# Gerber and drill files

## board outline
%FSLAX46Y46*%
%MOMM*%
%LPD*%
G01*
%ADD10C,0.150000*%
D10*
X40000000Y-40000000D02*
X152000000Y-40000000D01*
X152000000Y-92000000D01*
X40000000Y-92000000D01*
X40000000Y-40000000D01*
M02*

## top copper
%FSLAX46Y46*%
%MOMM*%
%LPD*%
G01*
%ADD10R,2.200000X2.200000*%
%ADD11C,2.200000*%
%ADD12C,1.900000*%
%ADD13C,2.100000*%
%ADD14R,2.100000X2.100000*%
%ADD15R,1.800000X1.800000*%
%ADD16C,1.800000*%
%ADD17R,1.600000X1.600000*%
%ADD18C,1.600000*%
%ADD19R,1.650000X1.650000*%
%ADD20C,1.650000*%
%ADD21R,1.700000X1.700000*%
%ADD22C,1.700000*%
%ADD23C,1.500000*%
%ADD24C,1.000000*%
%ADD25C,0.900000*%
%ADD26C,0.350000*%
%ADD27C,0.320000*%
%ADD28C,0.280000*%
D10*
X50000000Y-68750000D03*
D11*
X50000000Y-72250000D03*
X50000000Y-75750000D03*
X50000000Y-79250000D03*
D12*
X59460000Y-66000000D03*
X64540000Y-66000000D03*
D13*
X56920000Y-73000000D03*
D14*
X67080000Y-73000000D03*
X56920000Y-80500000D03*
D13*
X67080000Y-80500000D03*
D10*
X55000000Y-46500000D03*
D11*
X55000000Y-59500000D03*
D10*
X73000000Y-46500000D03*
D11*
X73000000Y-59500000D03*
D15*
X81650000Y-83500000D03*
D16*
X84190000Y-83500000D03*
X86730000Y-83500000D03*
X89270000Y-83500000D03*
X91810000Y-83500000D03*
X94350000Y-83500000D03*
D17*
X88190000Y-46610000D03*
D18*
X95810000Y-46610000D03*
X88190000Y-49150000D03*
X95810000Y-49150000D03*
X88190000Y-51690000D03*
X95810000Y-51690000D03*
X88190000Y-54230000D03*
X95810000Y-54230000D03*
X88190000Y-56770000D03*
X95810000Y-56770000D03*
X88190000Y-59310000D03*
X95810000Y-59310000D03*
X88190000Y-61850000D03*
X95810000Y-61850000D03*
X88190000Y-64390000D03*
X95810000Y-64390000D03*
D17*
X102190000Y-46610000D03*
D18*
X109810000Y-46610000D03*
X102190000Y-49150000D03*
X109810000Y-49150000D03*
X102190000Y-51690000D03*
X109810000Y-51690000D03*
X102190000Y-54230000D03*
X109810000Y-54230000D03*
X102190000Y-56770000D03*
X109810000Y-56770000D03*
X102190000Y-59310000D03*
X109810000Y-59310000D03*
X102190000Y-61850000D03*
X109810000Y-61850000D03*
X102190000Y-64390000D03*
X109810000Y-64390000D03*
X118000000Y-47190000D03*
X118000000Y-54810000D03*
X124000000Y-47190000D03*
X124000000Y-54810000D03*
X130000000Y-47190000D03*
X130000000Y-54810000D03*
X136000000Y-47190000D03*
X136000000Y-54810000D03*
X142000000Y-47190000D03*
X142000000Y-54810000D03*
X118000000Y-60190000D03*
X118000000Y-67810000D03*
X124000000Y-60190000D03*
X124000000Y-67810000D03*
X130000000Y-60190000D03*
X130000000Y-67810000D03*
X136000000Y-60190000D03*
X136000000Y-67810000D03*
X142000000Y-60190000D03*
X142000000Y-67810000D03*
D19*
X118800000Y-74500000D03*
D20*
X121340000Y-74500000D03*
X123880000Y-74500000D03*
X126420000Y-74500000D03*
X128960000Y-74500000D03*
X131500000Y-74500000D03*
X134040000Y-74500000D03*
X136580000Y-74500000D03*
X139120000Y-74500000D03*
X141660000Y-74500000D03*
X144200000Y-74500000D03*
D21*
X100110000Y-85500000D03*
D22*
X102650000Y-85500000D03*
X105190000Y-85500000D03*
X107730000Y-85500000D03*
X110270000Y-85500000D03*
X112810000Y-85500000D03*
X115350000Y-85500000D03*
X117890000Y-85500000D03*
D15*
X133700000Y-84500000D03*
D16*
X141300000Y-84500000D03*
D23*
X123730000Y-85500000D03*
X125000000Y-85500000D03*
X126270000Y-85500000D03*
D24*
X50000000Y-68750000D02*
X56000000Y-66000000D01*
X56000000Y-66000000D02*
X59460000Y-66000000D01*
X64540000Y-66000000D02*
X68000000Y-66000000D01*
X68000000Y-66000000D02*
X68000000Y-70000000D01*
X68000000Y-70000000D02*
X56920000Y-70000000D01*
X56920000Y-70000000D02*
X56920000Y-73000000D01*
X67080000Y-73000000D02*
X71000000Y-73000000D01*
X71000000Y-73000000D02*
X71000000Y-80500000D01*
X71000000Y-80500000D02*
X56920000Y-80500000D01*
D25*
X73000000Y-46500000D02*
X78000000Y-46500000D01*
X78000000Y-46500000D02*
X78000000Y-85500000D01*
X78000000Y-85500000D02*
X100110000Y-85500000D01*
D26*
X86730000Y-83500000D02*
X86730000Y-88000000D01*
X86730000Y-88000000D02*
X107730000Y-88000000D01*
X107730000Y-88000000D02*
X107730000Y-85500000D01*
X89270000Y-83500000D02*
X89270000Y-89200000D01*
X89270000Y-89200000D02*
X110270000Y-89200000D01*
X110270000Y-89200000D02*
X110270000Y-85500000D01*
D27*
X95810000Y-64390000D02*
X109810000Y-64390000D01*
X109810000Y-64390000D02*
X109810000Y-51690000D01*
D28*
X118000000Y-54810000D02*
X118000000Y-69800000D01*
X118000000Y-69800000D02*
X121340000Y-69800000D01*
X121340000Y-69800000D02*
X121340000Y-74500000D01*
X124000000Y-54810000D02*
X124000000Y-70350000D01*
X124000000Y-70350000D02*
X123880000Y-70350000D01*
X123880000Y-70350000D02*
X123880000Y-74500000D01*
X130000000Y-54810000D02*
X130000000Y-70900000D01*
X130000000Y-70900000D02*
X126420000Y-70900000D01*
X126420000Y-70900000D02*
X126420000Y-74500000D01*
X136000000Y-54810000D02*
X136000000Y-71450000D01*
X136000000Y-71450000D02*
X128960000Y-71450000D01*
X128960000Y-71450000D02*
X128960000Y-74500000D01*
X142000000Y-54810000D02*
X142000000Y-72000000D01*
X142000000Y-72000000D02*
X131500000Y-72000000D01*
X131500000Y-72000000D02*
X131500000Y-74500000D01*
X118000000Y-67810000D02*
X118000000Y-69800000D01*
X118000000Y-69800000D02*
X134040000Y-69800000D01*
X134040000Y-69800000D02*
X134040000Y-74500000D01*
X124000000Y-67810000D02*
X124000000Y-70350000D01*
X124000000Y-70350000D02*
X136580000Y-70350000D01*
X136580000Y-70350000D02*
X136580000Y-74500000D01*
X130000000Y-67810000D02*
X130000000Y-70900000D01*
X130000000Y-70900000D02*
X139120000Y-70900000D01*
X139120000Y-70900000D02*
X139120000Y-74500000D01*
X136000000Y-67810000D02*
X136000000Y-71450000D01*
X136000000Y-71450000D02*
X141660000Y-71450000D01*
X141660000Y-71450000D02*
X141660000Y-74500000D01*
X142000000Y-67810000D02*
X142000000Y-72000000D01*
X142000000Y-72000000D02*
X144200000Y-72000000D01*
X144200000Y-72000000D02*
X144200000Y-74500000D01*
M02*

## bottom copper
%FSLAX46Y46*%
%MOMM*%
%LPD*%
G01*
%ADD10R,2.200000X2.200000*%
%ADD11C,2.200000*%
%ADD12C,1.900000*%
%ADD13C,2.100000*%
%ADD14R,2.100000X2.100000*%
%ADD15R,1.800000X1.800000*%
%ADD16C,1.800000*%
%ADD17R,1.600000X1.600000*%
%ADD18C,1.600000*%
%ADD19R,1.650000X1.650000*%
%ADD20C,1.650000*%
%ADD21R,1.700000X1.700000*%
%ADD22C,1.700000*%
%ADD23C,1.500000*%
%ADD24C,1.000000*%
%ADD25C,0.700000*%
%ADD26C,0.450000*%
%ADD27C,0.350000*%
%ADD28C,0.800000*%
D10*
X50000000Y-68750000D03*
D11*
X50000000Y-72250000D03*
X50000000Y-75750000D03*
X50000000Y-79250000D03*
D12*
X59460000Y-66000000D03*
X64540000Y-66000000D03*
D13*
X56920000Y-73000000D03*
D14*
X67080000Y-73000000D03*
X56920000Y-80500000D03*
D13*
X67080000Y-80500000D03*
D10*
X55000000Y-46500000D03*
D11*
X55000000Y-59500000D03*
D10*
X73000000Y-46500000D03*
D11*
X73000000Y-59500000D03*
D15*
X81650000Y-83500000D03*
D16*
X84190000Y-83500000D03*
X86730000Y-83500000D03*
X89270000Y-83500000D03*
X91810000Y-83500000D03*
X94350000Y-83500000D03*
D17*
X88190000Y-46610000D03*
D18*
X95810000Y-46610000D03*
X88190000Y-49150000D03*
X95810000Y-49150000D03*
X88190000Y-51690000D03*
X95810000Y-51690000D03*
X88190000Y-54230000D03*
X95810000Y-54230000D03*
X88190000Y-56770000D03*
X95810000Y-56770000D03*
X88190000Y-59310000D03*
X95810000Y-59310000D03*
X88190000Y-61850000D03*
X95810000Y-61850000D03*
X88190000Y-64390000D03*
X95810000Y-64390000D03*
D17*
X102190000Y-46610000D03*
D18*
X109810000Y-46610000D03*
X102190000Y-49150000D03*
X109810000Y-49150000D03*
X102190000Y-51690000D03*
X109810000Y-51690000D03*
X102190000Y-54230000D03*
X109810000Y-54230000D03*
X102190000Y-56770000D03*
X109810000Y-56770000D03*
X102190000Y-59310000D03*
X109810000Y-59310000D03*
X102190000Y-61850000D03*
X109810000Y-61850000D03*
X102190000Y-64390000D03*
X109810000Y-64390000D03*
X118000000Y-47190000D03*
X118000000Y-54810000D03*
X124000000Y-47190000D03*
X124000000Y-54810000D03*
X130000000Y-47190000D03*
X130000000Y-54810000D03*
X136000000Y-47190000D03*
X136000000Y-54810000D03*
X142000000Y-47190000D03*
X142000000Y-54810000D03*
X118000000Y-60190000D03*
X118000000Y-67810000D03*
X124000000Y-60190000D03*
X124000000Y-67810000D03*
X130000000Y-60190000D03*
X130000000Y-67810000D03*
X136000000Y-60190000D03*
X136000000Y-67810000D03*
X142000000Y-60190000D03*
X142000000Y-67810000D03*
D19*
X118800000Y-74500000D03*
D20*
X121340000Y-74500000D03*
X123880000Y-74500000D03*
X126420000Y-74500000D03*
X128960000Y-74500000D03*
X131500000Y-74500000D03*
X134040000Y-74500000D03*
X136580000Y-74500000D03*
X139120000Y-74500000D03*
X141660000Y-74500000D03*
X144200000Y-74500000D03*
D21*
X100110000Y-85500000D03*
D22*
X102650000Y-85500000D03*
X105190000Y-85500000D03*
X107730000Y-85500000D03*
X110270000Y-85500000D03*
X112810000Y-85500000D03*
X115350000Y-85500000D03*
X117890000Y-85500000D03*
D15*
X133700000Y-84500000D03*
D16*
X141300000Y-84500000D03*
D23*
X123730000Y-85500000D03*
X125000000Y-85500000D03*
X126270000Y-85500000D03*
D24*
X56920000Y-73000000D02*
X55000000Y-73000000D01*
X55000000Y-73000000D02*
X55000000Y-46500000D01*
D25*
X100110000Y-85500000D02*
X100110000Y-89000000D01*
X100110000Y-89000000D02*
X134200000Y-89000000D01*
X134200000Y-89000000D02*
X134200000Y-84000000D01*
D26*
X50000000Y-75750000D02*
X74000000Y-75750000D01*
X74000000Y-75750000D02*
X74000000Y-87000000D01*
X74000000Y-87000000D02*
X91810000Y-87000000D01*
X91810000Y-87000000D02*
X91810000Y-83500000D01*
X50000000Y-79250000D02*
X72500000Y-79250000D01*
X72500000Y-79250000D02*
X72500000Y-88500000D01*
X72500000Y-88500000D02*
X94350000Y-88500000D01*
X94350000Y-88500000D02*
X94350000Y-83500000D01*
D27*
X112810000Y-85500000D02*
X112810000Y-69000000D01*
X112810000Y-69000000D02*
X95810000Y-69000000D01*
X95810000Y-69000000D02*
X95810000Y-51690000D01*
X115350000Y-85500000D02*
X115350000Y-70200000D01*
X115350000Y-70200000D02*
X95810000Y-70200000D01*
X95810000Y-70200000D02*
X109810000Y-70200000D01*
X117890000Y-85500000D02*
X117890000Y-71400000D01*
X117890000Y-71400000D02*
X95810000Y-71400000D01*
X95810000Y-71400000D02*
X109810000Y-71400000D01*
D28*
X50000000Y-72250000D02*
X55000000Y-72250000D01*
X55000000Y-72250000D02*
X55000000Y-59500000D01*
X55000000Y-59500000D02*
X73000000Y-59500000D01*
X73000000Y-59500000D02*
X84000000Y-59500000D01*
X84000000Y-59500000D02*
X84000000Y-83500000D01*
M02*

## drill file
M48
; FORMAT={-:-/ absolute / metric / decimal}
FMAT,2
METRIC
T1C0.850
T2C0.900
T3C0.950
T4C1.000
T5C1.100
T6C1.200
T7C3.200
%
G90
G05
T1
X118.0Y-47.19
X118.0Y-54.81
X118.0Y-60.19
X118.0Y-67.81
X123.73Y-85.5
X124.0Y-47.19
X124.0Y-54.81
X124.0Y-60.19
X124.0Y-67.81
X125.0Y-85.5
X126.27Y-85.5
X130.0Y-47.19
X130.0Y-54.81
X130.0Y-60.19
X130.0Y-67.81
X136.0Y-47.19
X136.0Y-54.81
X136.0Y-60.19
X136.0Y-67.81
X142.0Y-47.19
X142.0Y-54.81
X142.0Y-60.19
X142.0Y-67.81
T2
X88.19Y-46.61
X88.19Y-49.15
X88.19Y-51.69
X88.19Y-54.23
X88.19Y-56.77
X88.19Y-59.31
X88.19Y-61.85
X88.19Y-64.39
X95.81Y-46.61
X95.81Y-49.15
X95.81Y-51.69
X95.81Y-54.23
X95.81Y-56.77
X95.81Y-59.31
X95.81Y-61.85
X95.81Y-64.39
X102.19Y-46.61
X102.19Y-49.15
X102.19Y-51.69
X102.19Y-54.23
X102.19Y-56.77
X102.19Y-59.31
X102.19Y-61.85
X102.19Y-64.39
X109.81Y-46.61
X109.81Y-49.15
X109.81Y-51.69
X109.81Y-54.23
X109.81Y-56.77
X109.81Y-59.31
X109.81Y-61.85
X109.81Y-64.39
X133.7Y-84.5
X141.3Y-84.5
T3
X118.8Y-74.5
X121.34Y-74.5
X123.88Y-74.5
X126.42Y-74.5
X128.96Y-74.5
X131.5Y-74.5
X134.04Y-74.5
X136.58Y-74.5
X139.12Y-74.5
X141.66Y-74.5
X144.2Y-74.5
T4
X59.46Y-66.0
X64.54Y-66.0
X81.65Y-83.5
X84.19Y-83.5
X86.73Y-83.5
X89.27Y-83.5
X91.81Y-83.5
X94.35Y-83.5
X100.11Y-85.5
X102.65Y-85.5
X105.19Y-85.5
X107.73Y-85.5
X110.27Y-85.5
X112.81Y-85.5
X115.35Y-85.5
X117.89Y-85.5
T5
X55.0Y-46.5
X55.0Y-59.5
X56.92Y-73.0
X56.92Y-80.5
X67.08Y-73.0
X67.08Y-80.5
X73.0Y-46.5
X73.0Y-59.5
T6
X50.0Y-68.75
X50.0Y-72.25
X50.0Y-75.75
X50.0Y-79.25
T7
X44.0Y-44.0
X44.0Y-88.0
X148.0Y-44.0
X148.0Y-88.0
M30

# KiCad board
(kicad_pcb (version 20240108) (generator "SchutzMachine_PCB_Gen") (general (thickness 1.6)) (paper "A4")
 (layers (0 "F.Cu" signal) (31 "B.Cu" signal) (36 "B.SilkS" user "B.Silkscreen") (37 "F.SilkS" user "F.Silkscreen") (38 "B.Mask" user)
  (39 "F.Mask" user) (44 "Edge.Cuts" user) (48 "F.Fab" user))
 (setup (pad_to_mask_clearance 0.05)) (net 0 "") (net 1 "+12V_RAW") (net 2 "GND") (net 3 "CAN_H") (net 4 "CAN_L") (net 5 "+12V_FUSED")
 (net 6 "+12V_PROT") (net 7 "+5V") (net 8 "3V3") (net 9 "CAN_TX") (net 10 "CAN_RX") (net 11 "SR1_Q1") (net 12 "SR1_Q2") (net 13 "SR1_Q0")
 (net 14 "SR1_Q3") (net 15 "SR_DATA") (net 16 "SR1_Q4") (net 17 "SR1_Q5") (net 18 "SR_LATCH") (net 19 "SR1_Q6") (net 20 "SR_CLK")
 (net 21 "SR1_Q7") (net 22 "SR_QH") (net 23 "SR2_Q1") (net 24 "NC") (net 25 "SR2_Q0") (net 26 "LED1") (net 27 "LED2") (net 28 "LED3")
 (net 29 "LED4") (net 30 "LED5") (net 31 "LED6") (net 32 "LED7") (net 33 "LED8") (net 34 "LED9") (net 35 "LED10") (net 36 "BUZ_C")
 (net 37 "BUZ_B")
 (gr_rect (start 40.0 40.0) (end 152.0 92.0) (stroke (width 0.15) (type solid)) (fill none) (layer "Edge.Cuts"))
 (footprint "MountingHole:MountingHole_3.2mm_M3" (layer "F.Cu") (at 44.0 44.0)
  (pad "" np_thru_hole circle (at 0 0) (size 3.2 3.2) (drill 3.2) (layers "*.Cu" "*.Mask")))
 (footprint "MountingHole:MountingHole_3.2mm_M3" (layer "F.Cu") (at 148.0 44.0)
  (pad "" np_thru_hole circle (at 0 0) (size 3.2 3.2) (drill 3.2) (layers "*.Cu" "*.Mask")))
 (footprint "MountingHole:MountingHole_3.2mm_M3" (layer "F.Cu") (at 44.0 88.0)
  (pad "" np_thru_hole circle (at 0 0) (size 3.2 3.2) (drill 3.2) (layers "*.Cu" "*.Mask")))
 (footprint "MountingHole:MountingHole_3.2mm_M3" (layer "F.Cu") (at 148.0 88.0)
  (pad "" np_thru_hole circle (at 0 0) (size 3.2 3.2) (drill 3.2) (layers "*.Cu" "*.Mask")))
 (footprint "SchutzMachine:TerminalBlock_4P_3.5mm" (layer "F.Cu") (at 50.0 74.0 0)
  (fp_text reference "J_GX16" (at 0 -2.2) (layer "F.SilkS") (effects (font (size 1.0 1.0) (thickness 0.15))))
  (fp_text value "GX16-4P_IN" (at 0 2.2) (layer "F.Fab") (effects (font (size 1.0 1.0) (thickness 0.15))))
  (pad "1" thru_hole rect (at 0 -5.25) (size 2.2 2.2) (drill 1.2) (layers "*.Cu" "*.Mask") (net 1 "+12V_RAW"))
  (pad "2" thru_hole circle (at 0 -1.75) (size 2.2 2.2) (drill 1.2) (layers "*.Cu" "*.Mask") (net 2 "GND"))
  (pad "3" thru_hole circle (at 0 1.75) (size 2.2 2.2) (drill 1.2) (layers "*.Cu" "*.Mask") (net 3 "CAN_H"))
  (pad "4" thru_hole circle (at 0 5.25) (size 2.2 2.2) (drill 1.2) (layers "*.Cu" "*.Mask") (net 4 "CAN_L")))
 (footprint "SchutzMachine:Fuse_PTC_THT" (layer "F.Cu") (at 62.0 66.0 0)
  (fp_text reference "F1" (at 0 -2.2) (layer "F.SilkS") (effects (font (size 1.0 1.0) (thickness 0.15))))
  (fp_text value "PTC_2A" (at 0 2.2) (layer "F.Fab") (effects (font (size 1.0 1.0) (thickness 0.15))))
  (pad "1" thru_hole circle (at -2.54 0) (size 1.9 1.9) (drill 1.0) (layers "*.Cu" "*.Mask") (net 1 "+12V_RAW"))
  (pad "2" thru_hole circle (at 2.54 0) (size 1.9 1.9) (drill 1.0) (layers "*.Cu" "*.Mask") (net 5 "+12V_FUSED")))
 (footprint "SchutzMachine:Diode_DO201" (layer "F.Cu") (at 62.0 73.0 0)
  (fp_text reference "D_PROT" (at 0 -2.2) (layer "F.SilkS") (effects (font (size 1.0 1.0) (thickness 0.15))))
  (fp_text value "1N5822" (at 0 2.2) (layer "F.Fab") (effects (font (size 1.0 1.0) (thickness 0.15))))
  (pad "1" thru_hole circle (at -5.08 0) (size 2.1 2.1) (drill 1.1) (layers "*.Cu" "*.Mask") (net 5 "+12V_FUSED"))
  (pad "2" thru_hole rect (at 5.08 0) (size 2.1 2.1) (drill 1.1) (layers "*.Cu" "*.Mask") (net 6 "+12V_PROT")))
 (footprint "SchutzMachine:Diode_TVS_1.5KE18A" (layer "F.Cu") (at 62.0 80.5 0)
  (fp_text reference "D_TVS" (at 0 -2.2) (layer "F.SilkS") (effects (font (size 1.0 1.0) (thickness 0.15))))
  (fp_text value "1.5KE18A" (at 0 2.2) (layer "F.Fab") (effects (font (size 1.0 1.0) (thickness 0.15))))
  (pad "1" thru_hole rect (at -5.08 0) (size 2.1 2.1) (drill 1.1) (layers "*.Cu" "*.Mask") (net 6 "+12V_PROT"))
  (pad "2" thru_hole circle (at 5.08 0) (size 2.1 2.1) (drill 1.1) (layers "*.Cu" "*.Mask") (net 2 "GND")))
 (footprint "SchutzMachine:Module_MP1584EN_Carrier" (layer "F.Cu") (at 64.0 53.0 0)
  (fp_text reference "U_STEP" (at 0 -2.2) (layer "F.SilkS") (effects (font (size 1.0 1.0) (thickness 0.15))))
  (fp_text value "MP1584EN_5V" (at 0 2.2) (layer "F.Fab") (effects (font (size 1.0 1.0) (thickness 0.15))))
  (pad "1" thru_hole rect (at -9.0 -6.5) (size 2.2 2.2) (drill 1.1) (layers "*.Cu" "*.Mask") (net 6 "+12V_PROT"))
  (pad "2" thru_hole circle (at -9.0 6.5) (size 2.2 2.2) (drill 1.1) (layers "*.Cu" "*.Mask") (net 2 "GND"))
  (pad "3" thru_hole rect (at 9.0 -6.5) (size 2.2 2.2) (drill 1.1) (layers "*.Cu" "*.Mask") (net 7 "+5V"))
  (pad "4" thru_hole circle (at 9.0 6.5) (size 2.2 2.2) (drill 1.1) (layers "*.Cu" "*.Mask") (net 2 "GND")))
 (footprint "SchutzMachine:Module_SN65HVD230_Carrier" (layer "F.Cu") (at 88.0 79.0 0)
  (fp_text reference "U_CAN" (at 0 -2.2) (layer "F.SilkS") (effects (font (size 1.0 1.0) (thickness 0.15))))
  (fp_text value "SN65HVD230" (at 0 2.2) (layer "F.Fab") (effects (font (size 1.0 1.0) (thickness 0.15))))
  (pad "1" thru_hole rect (at -6.35 4.5) (size 1.8 1.8) (drill 1.0) (layers "*.Cu" "*.Mask") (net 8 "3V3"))
  (pad "2" thru_hole circle (at -3.81 4.5) (size 1.8 1.8) (drill 1.0) (layers "*.Cu" "*.Mask") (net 2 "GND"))
  (pad "3" thru_hole circle (at -1.27 4.5) (size 1.8 1.8) (drill 1.0) (layers "*.Cu" "*.Mask") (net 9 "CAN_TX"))
  (pad "4" thru_hole circle (at 1.27 4.5) (size 1.8 1.8) (drill 1.0) (layers "*.Cu" "*.Mask") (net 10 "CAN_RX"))
  (pad "5" thru_hole circle (at 3.81 4.5) (size 1.8 1.8) (drill 1.0) (layers "*.Cu" "*.Mask") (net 3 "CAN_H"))
  (pad "6" thru_hole circle (at 6.35 4.5) (size 1.8 1.8) (drill 1.0) (layers "*.Cu" "*.Mask") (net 4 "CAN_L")))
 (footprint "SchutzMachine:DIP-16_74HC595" (layer "F.Cu") (at 92.0 55.5 0)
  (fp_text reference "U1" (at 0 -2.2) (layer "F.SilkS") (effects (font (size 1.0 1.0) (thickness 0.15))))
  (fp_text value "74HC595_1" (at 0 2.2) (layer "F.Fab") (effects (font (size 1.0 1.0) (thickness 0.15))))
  (pad "1" thru_hole rect (at -3.81 -8.89) (size 1.6 1.6) (drill 0.9) (layers "*.Cu" "*.Mask") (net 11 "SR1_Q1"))
  (pad "16" thru_hole circle (at 3.81 -8.89) (size 1.6 1.6) (drill 0.9) (layers "*.Cu" "*.Mask") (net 8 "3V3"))
  (pad "2" thru_hole circle (at -3.81 -6.35) (size 1.6 1.6) (drill 0.9) (layers "*.Cu" "*.Mask") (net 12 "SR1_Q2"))
  (pad "15" thru_hole circle (at 3.81 -6.35) (size 1.6 1.6) (drill 0.9) (layers "*.Cu" "*.Mask") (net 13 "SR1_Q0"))
  (pad "3" thru_hole circle (at -3.81 -3.81) (size 1.6 1.6) (drill 0.9) (layers "*.Cu" "*.Mask") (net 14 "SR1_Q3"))
  (pad "14" thru_hole circle (at 3.81 -3.81) (size 1.6 1.6) (drill 0.9) (layers "*.Cu" "*.Mask") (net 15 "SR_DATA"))
  (pad "4" thru_hole circle (at -3.81 -1.27) (size 1.6 1.6) (drill 0.9) (layers "*.Cu" "*.Mask") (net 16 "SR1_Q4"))
  (pad "13" thru_hole circle (at 3.81 -1.27) (size 1.6 1.6) (drill 0.9) (layers "*.Cu" "*.Mask") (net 2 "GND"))
  (pad "5" thru_hole circle (at -3.81 1.27) (size 1.6 1.6) (drill 0.9) (layers "*.Cu" "*.Mask") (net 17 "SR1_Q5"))
  (pad "12" thru_hole circle (at 3.81 1.27) (size 1.6 1.6) (drill 0.9) (layers "*.Cu" "*.Mask") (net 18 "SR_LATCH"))
  (pad "6" thru_hole circle (at -3.81 3.81) (size 1.6 1.6) (drill 0.9) (layers "*.Cu" "*.Mask") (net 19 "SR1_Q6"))
  (pad "11" thru_hole circle (at 3.81 3.81) (size 1.6 1.6) (drill 0.9) (layers "*.Cu" "*.Mask") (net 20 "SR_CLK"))
  (pad "7" thru_hole circle (at -3.81 6.35) (size 1.6 1.6) (drill 0.9) (layers "*.Cu" "*.Mask") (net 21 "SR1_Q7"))
  (pad "10" thru_hole circle (at 3.81 6.35) (size 1.6 1.6) (drill 0.9) (layers "*.Cu" "*.Mask") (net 8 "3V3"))
  (pad "8" thru_hole circle (at -3.81 8.89) (size 1.6 1.6) (drill 0.9) (layers "*.Cu" "*.Mask") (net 2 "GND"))
  (pad "9" thru_hole circle (at 3.81 8.89) (size 1.6 1.6) (drill 0.9) (layers "*.Cu" "*.Mask") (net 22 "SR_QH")))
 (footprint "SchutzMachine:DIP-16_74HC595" (layer "F.Cu") (at 106.0 55.5 0)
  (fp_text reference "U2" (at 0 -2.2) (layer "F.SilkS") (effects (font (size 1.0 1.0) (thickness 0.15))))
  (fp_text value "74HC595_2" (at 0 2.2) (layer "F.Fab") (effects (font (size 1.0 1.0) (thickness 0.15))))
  (pad "1" thru_hole rect (at -3.81 -8.89) (size 1.6 1.6) (drill 0.9) (layers "*.Cu" "*.Mask") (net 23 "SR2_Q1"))
  (pad "16" thru_hole circle (at 3.81 -8.89) (size 1.6 1.6) (drill 0.9) (layers "*.Cu" "*.Mask") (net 8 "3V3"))
  (pad "2" thru_hole circle (at -3.81 -6.35) (size 1.6 1.6) (drill 0.9) (layers "*.Cu" "*.Mask") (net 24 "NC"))
  (pad "15" thru_hole circle (at 3.81 -6.35) (size 1.6 1.6) (drill 0.9) (layers "*.Cu" "*.Mask") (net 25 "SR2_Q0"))
  (pad "3" thru_hole circle (at -3.81 -3.81) (size 1.6 1.6) (drill 0.9) (layers "*.Cu" "*.Mask") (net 24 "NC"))
  (pad "14" thru_hole circle (at 3.81 -3.81) (size 1.6 1.6) (drill 0.9) (layers "*.Cu" "*.Mask") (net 22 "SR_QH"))
  (pad "4" thru_hole circle (at -3.81 -1.27) (size 1.6 1.6) (drill 0.9) (layers "*.Cu" "*.Mask") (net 24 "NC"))
  (pad "13" thru_hole circle (at 3.81 -1.27) (size 1.6 1.6) (drill 0.9) (layers "*.Cu" "*.Mask") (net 2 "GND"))
  (pad "5" thru_hole circle (at -3.81 1.27) (size 1.6 1.6) (drill 0.9) (layers "*.Cu" "*.Mask") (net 24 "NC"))
  (pad "12" thru_hole circle (at 3.81 1.27) (size 1.6 1.6) (drill 0.9) (layers "*.Cu" "*.Mask") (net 18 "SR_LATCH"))
  (pad "6" thru_hole circle (at -3.81 3.81) (size 1.6 1.6) (drill 0.9) (layers "*.Cu" "*.Mask") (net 24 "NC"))
  (pad "11" thru_hole circle (at 3.81 3.81) (size 1.6 1.6) (drill 0.9) (layers "*.Cu" "*.Mask") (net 20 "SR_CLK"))
  (pad "7" thru_hole circle (at -3.81 6.35) (size 1.6 1.6) (drill 0.9) (layers "*.Cu" "*.Mask") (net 24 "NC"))
  (pad "10" thru_hole circle (at 3.81 6.35) (size 1.6 1.6) (drill 0.9) (layers "*.Cu" "*.Mask") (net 8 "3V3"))
  (pad "8" thru_hole circle (at -3.81 8.89) (size 1.6 1.6) (drill 0.9) (layers "*.Cu" "*.Mask") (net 2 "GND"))
  (pad "9" thru_hole circle (at 3.81 8.89) (size 1.6 1.6) (drill 0.9) (layers "*.Cu" "*.Mask") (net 24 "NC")))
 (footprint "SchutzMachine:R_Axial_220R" (layer "F.Cu") (at 118.0 51.0 0)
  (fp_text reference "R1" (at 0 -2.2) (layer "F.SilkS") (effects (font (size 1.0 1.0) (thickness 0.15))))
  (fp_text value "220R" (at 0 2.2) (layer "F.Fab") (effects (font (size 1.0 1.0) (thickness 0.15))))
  (pad "1" thru_hole circle (at 0 -3.81) (size 1.6 1.6) (drill 0.85) (layers "*.Cu" "*.Mask") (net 13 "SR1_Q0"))
  (pad "2" thru_hole circle (at 0 3.81) (size 1.6 1.6) (drill 0.85) (layers "*.Cu" "*.Mask") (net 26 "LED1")))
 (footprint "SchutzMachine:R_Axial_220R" (layer "F.Cu") (at 124.0 51.0 0)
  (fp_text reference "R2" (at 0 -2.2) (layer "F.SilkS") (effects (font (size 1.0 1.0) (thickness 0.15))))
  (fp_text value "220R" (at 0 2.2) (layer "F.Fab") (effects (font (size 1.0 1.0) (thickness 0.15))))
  (pad "1" thru_hole circle (at 0 -3.81) (size 1.6 1.6) (drill 0.85) (layers "*.Cu" "*.Mask") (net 11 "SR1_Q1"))
  (pad "2" thru_hole circle (at 0 3.81) (size 1.6 1.6) (drill 0.85) (layers "*.Cu" "*.Mask") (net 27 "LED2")))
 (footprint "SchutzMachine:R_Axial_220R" (layer "F.Cu") (at 130.0 51.0 0)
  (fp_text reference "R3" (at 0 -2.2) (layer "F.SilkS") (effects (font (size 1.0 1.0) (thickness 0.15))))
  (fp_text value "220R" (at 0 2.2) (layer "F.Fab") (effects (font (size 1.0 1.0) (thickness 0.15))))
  (pad "1" thru_hole circle (at 0 -3.81) (size 1.6 1.6) (drill 0.85) (layers "*.Cu" "*.Mask") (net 12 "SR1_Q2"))
  (pad "2" thru_hole circle (at 0 3.81) (size 1.6 1.6) (drill 0.85) (layers "*.Cu" "*.Mask") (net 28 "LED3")))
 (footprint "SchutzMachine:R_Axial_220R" (layer "F.Cu") (at 136.0 51.0 0)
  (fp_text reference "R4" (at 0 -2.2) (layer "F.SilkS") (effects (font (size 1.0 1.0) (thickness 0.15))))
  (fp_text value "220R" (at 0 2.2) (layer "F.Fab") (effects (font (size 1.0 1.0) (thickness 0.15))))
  (pad "1" thru_hole circle (at 0 -3.81) (size 1.6 1.6) (drill 0.85) (layers "*.Cu" "*.Mask") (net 14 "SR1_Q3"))
  (pad "2" thru_hole circle (at 0 3.81) (size 1.6 1.6) (drill 0.85) (layers "*.Cu" "*.Mask") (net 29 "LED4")))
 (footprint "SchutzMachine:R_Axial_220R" (layer "F.Cu") (at 142.0 51.0 0)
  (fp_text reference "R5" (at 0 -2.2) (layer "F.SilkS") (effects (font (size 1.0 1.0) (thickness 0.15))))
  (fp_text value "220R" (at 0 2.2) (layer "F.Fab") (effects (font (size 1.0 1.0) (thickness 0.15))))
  (pad "1" thru_hole circle (at 0 -3.81) (size 1.6 1.6) (drill 0.85) (layers "*.Cu" "*.Mask") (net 16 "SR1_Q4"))
  (pad "2" thru_hole circle (at 0 3.81) (size 1.6 1.6) (drill 0.85) (layers "*.Cu" "*.Mask") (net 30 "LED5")))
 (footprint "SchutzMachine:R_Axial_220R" (layer "F.Cu") (at 118.0 64.0 0)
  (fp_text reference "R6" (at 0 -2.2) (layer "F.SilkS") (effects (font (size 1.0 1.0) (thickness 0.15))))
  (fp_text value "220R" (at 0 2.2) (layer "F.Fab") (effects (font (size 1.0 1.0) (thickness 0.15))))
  (pad "1" thru_hole circle (at 0 -3.81) (size 1.6 1.6) (drill 0.85) (layers "*.Cu" "*.Mask") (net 17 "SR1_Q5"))
  (pad "2" thru_hole circle (at 0 3.81) (size 1.6 1.6) (drill 0.85) (layers "*.Cu" "*.Mask") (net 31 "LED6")))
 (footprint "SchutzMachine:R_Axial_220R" (layer "F.Cu") (at 124.0 64.0 0)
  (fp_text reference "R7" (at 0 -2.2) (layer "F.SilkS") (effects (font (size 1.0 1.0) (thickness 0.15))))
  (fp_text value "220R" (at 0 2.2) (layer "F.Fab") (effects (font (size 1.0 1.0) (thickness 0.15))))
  (pad "1" thru_hole circle (at 0 -3.81) (size 1.6 1.6) (drill 0.85) (layers "*.Cu" "*.Mask") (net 19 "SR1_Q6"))
  (pad "2" thru_hole circle (at 0 3.81) (size 1.6 1.6) (drill 0.85) (layers "*.Cu" "*.Mask") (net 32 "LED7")))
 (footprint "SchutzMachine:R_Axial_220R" (layer "F.Cu") (at 130.0 64.0 0)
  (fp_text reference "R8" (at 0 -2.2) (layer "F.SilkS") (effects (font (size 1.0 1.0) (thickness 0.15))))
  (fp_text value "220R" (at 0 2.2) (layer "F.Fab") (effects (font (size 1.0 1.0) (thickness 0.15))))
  (pad "1" thru_hole circle (at 0 -3.81) (size 1.6 1.6) (drill 0.85) (layers "*.Cu" "*.Mask") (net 21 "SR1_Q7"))
  (pad "2" thru_hole circle (at 0 3.81) (size 1.6 1.6) (drill 0.85) (layers "*.Cu" "*.Mask") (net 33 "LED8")))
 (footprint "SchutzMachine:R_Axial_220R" (layer "F.Cu") (at 136.0 64.0 0)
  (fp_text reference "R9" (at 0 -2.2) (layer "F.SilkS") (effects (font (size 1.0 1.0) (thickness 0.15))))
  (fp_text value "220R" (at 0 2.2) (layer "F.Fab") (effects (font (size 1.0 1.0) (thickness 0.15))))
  (pad "1" thru_hole circle (at 0 -3.81) (size 1.6 1.6) (drill 0.85) (layers "*.Cu" "*.Mask") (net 25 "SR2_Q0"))
  (pad "2" thru_hole circle (at 0 3.81) (size 1.6 1.6) (drill 0.85) (layers "*.Cu" "*.Mask") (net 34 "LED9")))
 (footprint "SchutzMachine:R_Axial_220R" (layer "F.Cu") (at 142.0 64.0 0)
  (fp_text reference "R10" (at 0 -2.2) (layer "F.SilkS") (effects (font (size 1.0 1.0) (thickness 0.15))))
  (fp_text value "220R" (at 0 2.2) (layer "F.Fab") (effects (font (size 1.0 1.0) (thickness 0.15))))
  (pad "1" thru_hole circle (at 0 -3.81) (size 1.6 1.6) (drill 0.85) (layers "*.Cu" "*.Mask") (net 23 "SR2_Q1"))
  (pad "2" thru_hole circle (at 0 3.81) (size 1.6 1.6) (drill 0.85) (layers "*.Cu" "*.Mask") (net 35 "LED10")))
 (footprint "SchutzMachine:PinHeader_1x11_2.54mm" (layer "F.Cu") (at 131.5 74.5 0)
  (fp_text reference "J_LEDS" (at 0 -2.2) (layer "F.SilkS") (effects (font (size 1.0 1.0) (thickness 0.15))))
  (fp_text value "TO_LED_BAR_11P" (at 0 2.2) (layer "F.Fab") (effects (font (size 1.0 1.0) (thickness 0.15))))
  (pad "1" thru_hole rect (at -12.7 0.0) (size 1.65 1.65) (drill 0.95) (layers "*.Cu" "*.Mask") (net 2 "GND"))
  (pad "2" thru_hole circle (at -10.16 0.0) (size 1.65 1.65) (drill 0.95) (layers "*.Cu" "*.Mask") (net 26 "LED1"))
  (pad "3" thru_hole circle (at -7.62 0.0) (size 1.65 1.65) (drill 0.95) (layers "*.Cu" "*.Mask") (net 27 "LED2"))
  (pad "4" thru_hole circle (at -5.08 0.0) (size 1.65 1.65) (drill 0.95) (layers "*.Cu" "*.Mask") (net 28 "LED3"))
  (pad "5" thru_hole circle (at -2.54 0.0) (size 1.65 1.65) (drill 0.95) (layers "*.Cu" "*.Mask") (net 29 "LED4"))
  (pad "6" thru_hole circle (at 0.0 0.0) (size 1.65 1.65) (drill 0.95) (layers "*.Cu" "*.Mask") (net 30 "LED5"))
  (pad "7" thru_hole circle (at 2.54 0.0) (size 1.65 1.65) (drill 0.95) (layers "*.Cu" "*.Mask") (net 31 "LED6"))
  (pad "8" thru_hole circle (at 5.08 0.0) (size 1.65 1.65) (drill 0.95) (layers "*.Cu" "*.Mask") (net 32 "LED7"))
  (pad "9" thru_hole circle (at 7.62 0.0) (size 1.65 1.65) (drill 0.95) (layers "*.Cu" "*.Mask") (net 33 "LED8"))
  (pad "10" thru_hole circle (at 10.16 0.0) (size 1.65 1.65) (drill 0.95) (layers "*.Cu" "*.Mask") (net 34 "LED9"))
  (pad "11" thru_hole circle (at 12.7 0.0) (size 1.65 1.65) (drill 0.95) (layers "*.Cu" "*.Mask") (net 35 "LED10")))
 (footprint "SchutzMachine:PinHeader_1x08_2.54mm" (layer "F.Cu") (at 109.0 85.5 0)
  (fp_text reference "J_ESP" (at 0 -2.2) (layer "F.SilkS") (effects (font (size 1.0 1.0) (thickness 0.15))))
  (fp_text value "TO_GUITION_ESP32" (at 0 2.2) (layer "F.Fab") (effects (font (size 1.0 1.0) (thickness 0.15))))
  (pad "1" thru_hole rect (at -8.89 0) (size 1.7 1.7) (drill 1.0) (layers "*.Cu" "*.Mask") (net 7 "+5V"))
  (pad "2" thru_hole circle (at -6.35 0) (size 1.7 1.7) (drill 1.0) (layers "*.Cu" "*.Mask") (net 8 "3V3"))
  (pad "3" thru_hole circle (at -3.81 0) (size 1.7 1.7) (drill 1.0) (layers "*.Cu" "*.Mask") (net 2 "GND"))
  (pad "4" thru_hole circle (at -1.27 0) (size 1.7 1.7) (drill 1.0) (layers "*.Cu" "*.Mask") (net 9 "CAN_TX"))
  (pad "5" thru_hole circle (at 1.27 0) (size 1.7 1.7) (drill 1.0) (layers "*.Cu" "*.Mask") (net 10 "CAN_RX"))
  (pad "6" thru_hole circle (at 3.81 0) (size 1.7 1.7) (drill 1.0) (layers "*.Cu" "*.Mask") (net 15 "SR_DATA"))
  (pad "7" thru_hole circle (at 6.35 0) (size 1.7 1.7) (drill 1.0) (layers "*.Cu" "*.Mask") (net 20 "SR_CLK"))
  (pad "8" thru_hole circle (at 8.89 0) (size 1.7 1.7) (drill 1.0) (layers "*.Cu" "*.Mask") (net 18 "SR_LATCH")))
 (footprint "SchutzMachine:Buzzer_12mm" (layer "F.Cu") (at 137.5 84.5 0)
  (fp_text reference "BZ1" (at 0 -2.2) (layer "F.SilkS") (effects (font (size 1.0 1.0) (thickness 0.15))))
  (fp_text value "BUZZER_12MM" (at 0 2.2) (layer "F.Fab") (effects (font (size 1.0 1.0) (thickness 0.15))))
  (pad "1" thru_hole rect (at -3.8 0) (size 1.8 1.8) (drill 0.9) (layers "*.Cu" "*.Mask") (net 7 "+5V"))
  (pad "2" thru_hole circle (at 3.8 0) (size 1.8 1.8) (drill 0.9) (layers "*.Cu" "*.Mask") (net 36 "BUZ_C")))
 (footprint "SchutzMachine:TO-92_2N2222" (layer "F.Cu") (at 125.0 85.5 0)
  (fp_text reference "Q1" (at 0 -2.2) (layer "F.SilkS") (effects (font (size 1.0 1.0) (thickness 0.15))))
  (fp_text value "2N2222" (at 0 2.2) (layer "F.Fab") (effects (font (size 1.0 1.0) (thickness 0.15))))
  (pad "1" thru_hole circle (at -1.27 0) (size 1.5 1.5) (drill 0.85) (layers "*.Cu" "*.Mask") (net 2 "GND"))
  (pad "2" thru_hole circle (at 0.0 0) (size 1.5 1.5) (drill 0.85) (layers "*.Cu" "*.Mask") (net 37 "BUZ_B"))
  (pad "3" thru_hole circle (at 1.27 0) (size 1.5 1.5) (drill 0.85) (layers "*.Cu" "*.Mask") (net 36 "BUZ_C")))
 (segment (start 50.0 68.75) (end 56.0 66.0) (width 1.0) (layer "F.Cu") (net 1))
 (segment (start 56.0 66.0) (end 59.46 66.0) (width 1.0) (layer "F.Cu") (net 1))
 (segment (start 64.54 66.0) (end 68.0 66.0) (width 1.0) (layer "F.Cu") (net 5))
 (segment (start 68.0 66.0) (end 68.0 70.0) (width 1.0) (layer "F.Cu") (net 5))
 (segment (start 68.0 70.0) (end 56.92 70.0) (width 1.0) (layer "F.Cu") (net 5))
 (segment (start 56.92 70.0) (end 56.92 73.0) (width 1.0) (layer "F.Cu") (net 5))
 (segment (start 67.08 73.0) (end 71.0 73.0) (width 1.0) (layer "F.Cu") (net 6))
 (segment (start 71.0 73.0) (end 71.0 80.5) (width 1.0) (layer "F.Cu") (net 6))
 (segment (start 71.0 80.5) (end 56.92 80.5) (width 1.0) (layer "F.Cu") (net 6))
 (segment (start 56.92 73.0) (end 55.0 73.0) (width 1.0) (layer "B.Cu") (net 6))
 (segment (start 55.0 73.0) (end 55.0 46.5) (width 1.0) (layer "B.Cu") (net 6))
 (segment (start 73.0 46.5) (end 78.0 46.5) (width 0.9) (layer "F.Cu") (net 7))
 (segment (start 78.0 46.5) (end 78.0 85.5) (width 0.9) (layer "F.Cu") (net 7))
 (segment (start 78.0 85.5) (end 100.11 85.5) (width 0.9) (layer "F.Cu") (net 7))
 (segment (start 100.11 85.5) (end 100.11 89.0) (width 0.7) (layer "B.Cu") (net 7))
 (segment (start 100.11 89.0) (end 134.2 89.0) (width 0.7) (layer "B.Cu") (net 7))
 (segment (start 134.2 89.0) (end 134.2 84.0) (width 0.7) (layer "B.Cu") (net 7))
 (segment (start 50.0 75.75) (end 74.0 75.75) (width 0.45) (layer "B.Cu") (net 3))
 (segment (start 74.0 75.75) (end 74.0 87.0) (width 0.45) (layer "B.Cu") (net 3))
 (segment (start 74.0 87.0) (end 91.81 87.0) (width 0.45) (layer "B.Cu") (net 3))
 (segment (start 91.81 87.0) (end 91.81 83.5) (width 0.45) (layer "B.Cu") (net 3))
 (segment (start 50.0 79.25) (end 72.5 79.25) (width 0.45) (layer "B.Cu") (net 4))
 (segment (start 72.5 79.25) (end 72.5 88.5) (width 0.45) (layer "B.Cu") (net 4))
 (segment (start 72.5 88.5) (end 94.35 88.5) (width 0.45) (layer "B.Cu") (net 4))
 (segment (start 94.35 88.5) (end 94.35 83.5) (width 0.45) (layer "B.Cu") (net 4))
 (segment (start 86.73 83.5) (end 86.73 88.0) (width 0.35) (layer "F.Cu") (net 9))
 (segment (start 86.73 88.0) (end 107.73 88.0) (width 0.35) (layer "F.Cu") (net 9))
 (segment (start 107.73 88.0) (end 107.73 85.5) (width 0.35) (layer "F.Cu") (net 9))
 (segment (start 89.27 83.5) (end 89.27 89.2) (width 0.35) (layer "F.Cu") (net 10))
 (segment (start 89.27 89.2) (end 110.27 89.2) (width 0.35) (layer "F.Cu") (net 10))
 (segment (start 110.27 89.2) (end 110.27 85.5) (width 0.35) (layer "F.Cu") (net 10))
 (segment (start 112.81 85.5) (end 112.81 69.0) (width 0.35) (layer "B.Cu") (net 15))
 (segment (start 112.81 69.0) (end 95.81 69.0) (width 0.35) (layer "B.Cu") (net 15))
 (segment (start 95.81 69.0) (end 95.81 51.69) (width 0.35) (layer "B.Cu") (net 15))
 (segment (start 115.35 85.5) (end 115.35 70.2) (width 0.35) (layer "B.Cu") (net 20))
 (segment (start 115.35 70.2) (end 95.81 70.2) (width 0.35) (layer "B.Cu") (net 20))
 (segment (start 95.81 70.2) (end 109.81 70.2) (width 0.35) (layer "B.Cu") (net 20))
 (segment (start 117.89 85.5) (end 117.89 71.4) (width 0.35) (layer "B.Cu") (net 18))
 (segment (start 117.89 71.4) (end 95.81 71.4) (width 0.35) (layer "B.Cu") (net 18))
 (segment (start 95.81 71.4) (end 109.81 71.4) (width 0.35) (layer "B.Cu") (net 18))
 (segment (start 95.81 64.39) (end 109.81 64.39) (width 0.32) (layer "F.Cu") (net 22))
 (segment (start 109.81 64.39) (end 109.81 51.69) (width 0.32) (layer "F.Cu") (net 22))
 (segment (start 118.0 54.81) (end 118.0 69.8) (width 0.28) (layer "F.Cu") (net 26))
 (segment (start 118.0 69.8) (end 121.34 69.8) (width 0.28) (layer "F.Cu") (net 26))
 (segment (start 121.34 69.8) (end 121.34 74.5) (width 0.28) (layer "F.Cu") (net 26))
 (segment (start 124.0 54.81) (end 124.0 70.35) (width 0.28) (layer "F.Cu") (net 27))
 (segment (start 124.0 70.35) (end 123.88 70.35) (width 0.28) (layer "F.Cu") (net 27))
 (segment (start 123.88 70.35) (end 123.88 74.5) (width 0.28) (layer "F.Cu") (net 27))
 (segment (start 130.0 54.81) (end 130.0 70.9) (width 0.28) (layer "F.Cu") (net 28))
 (segment (start 130.0 70.9) (end 126.42 70.9) (width 0.28) (layer "F.Cu") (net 28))
 (segment (start 126.42 70.9) (end 126.42 74.5) (width 0.28) (layer "F.Cu") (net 28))
 (segment (start 136.0 54.81) (end 136.0 71.45) (width 0.28) (layer "F.Cu") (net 29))
 (segment (start 136.0 71.45) (end 128.96 71.45) (width 0.28) (layer "F.Cu") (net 29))
 (segment (start 128.96 71.45) (end 128.96 74.5) (width 0.28) (layer "F.Cu") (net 29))
 (segment (start 142.0 54.81) (end 142.0 72.0) (width 0.28) (layer "F.Cu") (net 30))
 (segment (start 142.0 72.0) (end 131.5 72.0) (width 0.28) (layer "F.Cu") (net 30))
 (segment (start 131.5 72.0) (end 131.5 74.5) (width 0.28) (layer "F.Cu") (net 30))
 (segment (start 118.0 67.81) (end 118.0 69.8) (width 0.28) (layer "F.Cu") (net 31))
 (segment (start 118.0 69.8) (end 134.04 69.8) (width 0.28) (layer "F.Cu") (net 31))
 (segment (start 134.04 69.8) (end 134.04 74.5) (width 0.28) (layer "F.Cu") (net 31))
 (segment (start 124.0 67.81) (end 124.0 70.35) (width 0.28) (layer "F.Cu") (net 32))
 (segment (start 124.0 70.35) (end 136.58 70.35) (width 0.28) (layer "F.Cu") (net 32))
 (segment (start 136.58 70.35) (end 136.58 74.5) (width 0.28) (layer "F.Cu") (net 32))
 (segment (start 130.0 67.81) (end 130.0 70.9) (width 0.28) (layer "F.Cu") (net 33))
 (segment (start 130.0 70.9) (end 139.12 70.9) (width 0.28) (layer "F.Cu") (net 33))
 (segment (start 139.12 70.9) (end 139.12 74.5) (width 0.28) (layer "F.Cu") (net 33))
 (segment (start 136.0 67.81) (end 136.0 71.45) (width 0.28) (layer "F.Cu") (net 34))
 (segment (start 136.0 71.45) (end 141.66 71.45) (width 0.28) (layer "F.Cu") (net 34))
 (segment (start 141.66 71.45) (end 141.66 74.5) (width 0.28) (layer "F.Cu") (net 34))
 (segment (start 142.0 67.81) (end 142.0 72.0) (width 0.28) (layer "F.Cu") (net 35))
 (segment (start 142.0 72.0) (end 144.2 72.0) (width 0.28) (layer "F.Cu") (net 35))
 (segment (start 144.2 72.0) (end 144.2 74.5) (width 0.28) (layer "F.Cu") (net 35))
 (segment (start 50.0 72.25) (end 55.0 72.25) (width 0.8) (layer "B.Cu") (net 2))
 (segment (start 55.0 72.25) (end 55.0 59.5) (width 0.8) (layer "B.Cu") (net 2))
 (segment (start 55.0 59.5) (end 73.0 59.5) (width 0.8) (layer "B.Cu") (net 2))
 (segment (start 73.0 59.5) (end 84.0 59.5) (width 0.8) (layer "B.Cu") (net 2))
 (segment (start 84.0 59.5) (end 84.0 83.5) (width 0.8) (layer "B.Cu") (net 2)))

